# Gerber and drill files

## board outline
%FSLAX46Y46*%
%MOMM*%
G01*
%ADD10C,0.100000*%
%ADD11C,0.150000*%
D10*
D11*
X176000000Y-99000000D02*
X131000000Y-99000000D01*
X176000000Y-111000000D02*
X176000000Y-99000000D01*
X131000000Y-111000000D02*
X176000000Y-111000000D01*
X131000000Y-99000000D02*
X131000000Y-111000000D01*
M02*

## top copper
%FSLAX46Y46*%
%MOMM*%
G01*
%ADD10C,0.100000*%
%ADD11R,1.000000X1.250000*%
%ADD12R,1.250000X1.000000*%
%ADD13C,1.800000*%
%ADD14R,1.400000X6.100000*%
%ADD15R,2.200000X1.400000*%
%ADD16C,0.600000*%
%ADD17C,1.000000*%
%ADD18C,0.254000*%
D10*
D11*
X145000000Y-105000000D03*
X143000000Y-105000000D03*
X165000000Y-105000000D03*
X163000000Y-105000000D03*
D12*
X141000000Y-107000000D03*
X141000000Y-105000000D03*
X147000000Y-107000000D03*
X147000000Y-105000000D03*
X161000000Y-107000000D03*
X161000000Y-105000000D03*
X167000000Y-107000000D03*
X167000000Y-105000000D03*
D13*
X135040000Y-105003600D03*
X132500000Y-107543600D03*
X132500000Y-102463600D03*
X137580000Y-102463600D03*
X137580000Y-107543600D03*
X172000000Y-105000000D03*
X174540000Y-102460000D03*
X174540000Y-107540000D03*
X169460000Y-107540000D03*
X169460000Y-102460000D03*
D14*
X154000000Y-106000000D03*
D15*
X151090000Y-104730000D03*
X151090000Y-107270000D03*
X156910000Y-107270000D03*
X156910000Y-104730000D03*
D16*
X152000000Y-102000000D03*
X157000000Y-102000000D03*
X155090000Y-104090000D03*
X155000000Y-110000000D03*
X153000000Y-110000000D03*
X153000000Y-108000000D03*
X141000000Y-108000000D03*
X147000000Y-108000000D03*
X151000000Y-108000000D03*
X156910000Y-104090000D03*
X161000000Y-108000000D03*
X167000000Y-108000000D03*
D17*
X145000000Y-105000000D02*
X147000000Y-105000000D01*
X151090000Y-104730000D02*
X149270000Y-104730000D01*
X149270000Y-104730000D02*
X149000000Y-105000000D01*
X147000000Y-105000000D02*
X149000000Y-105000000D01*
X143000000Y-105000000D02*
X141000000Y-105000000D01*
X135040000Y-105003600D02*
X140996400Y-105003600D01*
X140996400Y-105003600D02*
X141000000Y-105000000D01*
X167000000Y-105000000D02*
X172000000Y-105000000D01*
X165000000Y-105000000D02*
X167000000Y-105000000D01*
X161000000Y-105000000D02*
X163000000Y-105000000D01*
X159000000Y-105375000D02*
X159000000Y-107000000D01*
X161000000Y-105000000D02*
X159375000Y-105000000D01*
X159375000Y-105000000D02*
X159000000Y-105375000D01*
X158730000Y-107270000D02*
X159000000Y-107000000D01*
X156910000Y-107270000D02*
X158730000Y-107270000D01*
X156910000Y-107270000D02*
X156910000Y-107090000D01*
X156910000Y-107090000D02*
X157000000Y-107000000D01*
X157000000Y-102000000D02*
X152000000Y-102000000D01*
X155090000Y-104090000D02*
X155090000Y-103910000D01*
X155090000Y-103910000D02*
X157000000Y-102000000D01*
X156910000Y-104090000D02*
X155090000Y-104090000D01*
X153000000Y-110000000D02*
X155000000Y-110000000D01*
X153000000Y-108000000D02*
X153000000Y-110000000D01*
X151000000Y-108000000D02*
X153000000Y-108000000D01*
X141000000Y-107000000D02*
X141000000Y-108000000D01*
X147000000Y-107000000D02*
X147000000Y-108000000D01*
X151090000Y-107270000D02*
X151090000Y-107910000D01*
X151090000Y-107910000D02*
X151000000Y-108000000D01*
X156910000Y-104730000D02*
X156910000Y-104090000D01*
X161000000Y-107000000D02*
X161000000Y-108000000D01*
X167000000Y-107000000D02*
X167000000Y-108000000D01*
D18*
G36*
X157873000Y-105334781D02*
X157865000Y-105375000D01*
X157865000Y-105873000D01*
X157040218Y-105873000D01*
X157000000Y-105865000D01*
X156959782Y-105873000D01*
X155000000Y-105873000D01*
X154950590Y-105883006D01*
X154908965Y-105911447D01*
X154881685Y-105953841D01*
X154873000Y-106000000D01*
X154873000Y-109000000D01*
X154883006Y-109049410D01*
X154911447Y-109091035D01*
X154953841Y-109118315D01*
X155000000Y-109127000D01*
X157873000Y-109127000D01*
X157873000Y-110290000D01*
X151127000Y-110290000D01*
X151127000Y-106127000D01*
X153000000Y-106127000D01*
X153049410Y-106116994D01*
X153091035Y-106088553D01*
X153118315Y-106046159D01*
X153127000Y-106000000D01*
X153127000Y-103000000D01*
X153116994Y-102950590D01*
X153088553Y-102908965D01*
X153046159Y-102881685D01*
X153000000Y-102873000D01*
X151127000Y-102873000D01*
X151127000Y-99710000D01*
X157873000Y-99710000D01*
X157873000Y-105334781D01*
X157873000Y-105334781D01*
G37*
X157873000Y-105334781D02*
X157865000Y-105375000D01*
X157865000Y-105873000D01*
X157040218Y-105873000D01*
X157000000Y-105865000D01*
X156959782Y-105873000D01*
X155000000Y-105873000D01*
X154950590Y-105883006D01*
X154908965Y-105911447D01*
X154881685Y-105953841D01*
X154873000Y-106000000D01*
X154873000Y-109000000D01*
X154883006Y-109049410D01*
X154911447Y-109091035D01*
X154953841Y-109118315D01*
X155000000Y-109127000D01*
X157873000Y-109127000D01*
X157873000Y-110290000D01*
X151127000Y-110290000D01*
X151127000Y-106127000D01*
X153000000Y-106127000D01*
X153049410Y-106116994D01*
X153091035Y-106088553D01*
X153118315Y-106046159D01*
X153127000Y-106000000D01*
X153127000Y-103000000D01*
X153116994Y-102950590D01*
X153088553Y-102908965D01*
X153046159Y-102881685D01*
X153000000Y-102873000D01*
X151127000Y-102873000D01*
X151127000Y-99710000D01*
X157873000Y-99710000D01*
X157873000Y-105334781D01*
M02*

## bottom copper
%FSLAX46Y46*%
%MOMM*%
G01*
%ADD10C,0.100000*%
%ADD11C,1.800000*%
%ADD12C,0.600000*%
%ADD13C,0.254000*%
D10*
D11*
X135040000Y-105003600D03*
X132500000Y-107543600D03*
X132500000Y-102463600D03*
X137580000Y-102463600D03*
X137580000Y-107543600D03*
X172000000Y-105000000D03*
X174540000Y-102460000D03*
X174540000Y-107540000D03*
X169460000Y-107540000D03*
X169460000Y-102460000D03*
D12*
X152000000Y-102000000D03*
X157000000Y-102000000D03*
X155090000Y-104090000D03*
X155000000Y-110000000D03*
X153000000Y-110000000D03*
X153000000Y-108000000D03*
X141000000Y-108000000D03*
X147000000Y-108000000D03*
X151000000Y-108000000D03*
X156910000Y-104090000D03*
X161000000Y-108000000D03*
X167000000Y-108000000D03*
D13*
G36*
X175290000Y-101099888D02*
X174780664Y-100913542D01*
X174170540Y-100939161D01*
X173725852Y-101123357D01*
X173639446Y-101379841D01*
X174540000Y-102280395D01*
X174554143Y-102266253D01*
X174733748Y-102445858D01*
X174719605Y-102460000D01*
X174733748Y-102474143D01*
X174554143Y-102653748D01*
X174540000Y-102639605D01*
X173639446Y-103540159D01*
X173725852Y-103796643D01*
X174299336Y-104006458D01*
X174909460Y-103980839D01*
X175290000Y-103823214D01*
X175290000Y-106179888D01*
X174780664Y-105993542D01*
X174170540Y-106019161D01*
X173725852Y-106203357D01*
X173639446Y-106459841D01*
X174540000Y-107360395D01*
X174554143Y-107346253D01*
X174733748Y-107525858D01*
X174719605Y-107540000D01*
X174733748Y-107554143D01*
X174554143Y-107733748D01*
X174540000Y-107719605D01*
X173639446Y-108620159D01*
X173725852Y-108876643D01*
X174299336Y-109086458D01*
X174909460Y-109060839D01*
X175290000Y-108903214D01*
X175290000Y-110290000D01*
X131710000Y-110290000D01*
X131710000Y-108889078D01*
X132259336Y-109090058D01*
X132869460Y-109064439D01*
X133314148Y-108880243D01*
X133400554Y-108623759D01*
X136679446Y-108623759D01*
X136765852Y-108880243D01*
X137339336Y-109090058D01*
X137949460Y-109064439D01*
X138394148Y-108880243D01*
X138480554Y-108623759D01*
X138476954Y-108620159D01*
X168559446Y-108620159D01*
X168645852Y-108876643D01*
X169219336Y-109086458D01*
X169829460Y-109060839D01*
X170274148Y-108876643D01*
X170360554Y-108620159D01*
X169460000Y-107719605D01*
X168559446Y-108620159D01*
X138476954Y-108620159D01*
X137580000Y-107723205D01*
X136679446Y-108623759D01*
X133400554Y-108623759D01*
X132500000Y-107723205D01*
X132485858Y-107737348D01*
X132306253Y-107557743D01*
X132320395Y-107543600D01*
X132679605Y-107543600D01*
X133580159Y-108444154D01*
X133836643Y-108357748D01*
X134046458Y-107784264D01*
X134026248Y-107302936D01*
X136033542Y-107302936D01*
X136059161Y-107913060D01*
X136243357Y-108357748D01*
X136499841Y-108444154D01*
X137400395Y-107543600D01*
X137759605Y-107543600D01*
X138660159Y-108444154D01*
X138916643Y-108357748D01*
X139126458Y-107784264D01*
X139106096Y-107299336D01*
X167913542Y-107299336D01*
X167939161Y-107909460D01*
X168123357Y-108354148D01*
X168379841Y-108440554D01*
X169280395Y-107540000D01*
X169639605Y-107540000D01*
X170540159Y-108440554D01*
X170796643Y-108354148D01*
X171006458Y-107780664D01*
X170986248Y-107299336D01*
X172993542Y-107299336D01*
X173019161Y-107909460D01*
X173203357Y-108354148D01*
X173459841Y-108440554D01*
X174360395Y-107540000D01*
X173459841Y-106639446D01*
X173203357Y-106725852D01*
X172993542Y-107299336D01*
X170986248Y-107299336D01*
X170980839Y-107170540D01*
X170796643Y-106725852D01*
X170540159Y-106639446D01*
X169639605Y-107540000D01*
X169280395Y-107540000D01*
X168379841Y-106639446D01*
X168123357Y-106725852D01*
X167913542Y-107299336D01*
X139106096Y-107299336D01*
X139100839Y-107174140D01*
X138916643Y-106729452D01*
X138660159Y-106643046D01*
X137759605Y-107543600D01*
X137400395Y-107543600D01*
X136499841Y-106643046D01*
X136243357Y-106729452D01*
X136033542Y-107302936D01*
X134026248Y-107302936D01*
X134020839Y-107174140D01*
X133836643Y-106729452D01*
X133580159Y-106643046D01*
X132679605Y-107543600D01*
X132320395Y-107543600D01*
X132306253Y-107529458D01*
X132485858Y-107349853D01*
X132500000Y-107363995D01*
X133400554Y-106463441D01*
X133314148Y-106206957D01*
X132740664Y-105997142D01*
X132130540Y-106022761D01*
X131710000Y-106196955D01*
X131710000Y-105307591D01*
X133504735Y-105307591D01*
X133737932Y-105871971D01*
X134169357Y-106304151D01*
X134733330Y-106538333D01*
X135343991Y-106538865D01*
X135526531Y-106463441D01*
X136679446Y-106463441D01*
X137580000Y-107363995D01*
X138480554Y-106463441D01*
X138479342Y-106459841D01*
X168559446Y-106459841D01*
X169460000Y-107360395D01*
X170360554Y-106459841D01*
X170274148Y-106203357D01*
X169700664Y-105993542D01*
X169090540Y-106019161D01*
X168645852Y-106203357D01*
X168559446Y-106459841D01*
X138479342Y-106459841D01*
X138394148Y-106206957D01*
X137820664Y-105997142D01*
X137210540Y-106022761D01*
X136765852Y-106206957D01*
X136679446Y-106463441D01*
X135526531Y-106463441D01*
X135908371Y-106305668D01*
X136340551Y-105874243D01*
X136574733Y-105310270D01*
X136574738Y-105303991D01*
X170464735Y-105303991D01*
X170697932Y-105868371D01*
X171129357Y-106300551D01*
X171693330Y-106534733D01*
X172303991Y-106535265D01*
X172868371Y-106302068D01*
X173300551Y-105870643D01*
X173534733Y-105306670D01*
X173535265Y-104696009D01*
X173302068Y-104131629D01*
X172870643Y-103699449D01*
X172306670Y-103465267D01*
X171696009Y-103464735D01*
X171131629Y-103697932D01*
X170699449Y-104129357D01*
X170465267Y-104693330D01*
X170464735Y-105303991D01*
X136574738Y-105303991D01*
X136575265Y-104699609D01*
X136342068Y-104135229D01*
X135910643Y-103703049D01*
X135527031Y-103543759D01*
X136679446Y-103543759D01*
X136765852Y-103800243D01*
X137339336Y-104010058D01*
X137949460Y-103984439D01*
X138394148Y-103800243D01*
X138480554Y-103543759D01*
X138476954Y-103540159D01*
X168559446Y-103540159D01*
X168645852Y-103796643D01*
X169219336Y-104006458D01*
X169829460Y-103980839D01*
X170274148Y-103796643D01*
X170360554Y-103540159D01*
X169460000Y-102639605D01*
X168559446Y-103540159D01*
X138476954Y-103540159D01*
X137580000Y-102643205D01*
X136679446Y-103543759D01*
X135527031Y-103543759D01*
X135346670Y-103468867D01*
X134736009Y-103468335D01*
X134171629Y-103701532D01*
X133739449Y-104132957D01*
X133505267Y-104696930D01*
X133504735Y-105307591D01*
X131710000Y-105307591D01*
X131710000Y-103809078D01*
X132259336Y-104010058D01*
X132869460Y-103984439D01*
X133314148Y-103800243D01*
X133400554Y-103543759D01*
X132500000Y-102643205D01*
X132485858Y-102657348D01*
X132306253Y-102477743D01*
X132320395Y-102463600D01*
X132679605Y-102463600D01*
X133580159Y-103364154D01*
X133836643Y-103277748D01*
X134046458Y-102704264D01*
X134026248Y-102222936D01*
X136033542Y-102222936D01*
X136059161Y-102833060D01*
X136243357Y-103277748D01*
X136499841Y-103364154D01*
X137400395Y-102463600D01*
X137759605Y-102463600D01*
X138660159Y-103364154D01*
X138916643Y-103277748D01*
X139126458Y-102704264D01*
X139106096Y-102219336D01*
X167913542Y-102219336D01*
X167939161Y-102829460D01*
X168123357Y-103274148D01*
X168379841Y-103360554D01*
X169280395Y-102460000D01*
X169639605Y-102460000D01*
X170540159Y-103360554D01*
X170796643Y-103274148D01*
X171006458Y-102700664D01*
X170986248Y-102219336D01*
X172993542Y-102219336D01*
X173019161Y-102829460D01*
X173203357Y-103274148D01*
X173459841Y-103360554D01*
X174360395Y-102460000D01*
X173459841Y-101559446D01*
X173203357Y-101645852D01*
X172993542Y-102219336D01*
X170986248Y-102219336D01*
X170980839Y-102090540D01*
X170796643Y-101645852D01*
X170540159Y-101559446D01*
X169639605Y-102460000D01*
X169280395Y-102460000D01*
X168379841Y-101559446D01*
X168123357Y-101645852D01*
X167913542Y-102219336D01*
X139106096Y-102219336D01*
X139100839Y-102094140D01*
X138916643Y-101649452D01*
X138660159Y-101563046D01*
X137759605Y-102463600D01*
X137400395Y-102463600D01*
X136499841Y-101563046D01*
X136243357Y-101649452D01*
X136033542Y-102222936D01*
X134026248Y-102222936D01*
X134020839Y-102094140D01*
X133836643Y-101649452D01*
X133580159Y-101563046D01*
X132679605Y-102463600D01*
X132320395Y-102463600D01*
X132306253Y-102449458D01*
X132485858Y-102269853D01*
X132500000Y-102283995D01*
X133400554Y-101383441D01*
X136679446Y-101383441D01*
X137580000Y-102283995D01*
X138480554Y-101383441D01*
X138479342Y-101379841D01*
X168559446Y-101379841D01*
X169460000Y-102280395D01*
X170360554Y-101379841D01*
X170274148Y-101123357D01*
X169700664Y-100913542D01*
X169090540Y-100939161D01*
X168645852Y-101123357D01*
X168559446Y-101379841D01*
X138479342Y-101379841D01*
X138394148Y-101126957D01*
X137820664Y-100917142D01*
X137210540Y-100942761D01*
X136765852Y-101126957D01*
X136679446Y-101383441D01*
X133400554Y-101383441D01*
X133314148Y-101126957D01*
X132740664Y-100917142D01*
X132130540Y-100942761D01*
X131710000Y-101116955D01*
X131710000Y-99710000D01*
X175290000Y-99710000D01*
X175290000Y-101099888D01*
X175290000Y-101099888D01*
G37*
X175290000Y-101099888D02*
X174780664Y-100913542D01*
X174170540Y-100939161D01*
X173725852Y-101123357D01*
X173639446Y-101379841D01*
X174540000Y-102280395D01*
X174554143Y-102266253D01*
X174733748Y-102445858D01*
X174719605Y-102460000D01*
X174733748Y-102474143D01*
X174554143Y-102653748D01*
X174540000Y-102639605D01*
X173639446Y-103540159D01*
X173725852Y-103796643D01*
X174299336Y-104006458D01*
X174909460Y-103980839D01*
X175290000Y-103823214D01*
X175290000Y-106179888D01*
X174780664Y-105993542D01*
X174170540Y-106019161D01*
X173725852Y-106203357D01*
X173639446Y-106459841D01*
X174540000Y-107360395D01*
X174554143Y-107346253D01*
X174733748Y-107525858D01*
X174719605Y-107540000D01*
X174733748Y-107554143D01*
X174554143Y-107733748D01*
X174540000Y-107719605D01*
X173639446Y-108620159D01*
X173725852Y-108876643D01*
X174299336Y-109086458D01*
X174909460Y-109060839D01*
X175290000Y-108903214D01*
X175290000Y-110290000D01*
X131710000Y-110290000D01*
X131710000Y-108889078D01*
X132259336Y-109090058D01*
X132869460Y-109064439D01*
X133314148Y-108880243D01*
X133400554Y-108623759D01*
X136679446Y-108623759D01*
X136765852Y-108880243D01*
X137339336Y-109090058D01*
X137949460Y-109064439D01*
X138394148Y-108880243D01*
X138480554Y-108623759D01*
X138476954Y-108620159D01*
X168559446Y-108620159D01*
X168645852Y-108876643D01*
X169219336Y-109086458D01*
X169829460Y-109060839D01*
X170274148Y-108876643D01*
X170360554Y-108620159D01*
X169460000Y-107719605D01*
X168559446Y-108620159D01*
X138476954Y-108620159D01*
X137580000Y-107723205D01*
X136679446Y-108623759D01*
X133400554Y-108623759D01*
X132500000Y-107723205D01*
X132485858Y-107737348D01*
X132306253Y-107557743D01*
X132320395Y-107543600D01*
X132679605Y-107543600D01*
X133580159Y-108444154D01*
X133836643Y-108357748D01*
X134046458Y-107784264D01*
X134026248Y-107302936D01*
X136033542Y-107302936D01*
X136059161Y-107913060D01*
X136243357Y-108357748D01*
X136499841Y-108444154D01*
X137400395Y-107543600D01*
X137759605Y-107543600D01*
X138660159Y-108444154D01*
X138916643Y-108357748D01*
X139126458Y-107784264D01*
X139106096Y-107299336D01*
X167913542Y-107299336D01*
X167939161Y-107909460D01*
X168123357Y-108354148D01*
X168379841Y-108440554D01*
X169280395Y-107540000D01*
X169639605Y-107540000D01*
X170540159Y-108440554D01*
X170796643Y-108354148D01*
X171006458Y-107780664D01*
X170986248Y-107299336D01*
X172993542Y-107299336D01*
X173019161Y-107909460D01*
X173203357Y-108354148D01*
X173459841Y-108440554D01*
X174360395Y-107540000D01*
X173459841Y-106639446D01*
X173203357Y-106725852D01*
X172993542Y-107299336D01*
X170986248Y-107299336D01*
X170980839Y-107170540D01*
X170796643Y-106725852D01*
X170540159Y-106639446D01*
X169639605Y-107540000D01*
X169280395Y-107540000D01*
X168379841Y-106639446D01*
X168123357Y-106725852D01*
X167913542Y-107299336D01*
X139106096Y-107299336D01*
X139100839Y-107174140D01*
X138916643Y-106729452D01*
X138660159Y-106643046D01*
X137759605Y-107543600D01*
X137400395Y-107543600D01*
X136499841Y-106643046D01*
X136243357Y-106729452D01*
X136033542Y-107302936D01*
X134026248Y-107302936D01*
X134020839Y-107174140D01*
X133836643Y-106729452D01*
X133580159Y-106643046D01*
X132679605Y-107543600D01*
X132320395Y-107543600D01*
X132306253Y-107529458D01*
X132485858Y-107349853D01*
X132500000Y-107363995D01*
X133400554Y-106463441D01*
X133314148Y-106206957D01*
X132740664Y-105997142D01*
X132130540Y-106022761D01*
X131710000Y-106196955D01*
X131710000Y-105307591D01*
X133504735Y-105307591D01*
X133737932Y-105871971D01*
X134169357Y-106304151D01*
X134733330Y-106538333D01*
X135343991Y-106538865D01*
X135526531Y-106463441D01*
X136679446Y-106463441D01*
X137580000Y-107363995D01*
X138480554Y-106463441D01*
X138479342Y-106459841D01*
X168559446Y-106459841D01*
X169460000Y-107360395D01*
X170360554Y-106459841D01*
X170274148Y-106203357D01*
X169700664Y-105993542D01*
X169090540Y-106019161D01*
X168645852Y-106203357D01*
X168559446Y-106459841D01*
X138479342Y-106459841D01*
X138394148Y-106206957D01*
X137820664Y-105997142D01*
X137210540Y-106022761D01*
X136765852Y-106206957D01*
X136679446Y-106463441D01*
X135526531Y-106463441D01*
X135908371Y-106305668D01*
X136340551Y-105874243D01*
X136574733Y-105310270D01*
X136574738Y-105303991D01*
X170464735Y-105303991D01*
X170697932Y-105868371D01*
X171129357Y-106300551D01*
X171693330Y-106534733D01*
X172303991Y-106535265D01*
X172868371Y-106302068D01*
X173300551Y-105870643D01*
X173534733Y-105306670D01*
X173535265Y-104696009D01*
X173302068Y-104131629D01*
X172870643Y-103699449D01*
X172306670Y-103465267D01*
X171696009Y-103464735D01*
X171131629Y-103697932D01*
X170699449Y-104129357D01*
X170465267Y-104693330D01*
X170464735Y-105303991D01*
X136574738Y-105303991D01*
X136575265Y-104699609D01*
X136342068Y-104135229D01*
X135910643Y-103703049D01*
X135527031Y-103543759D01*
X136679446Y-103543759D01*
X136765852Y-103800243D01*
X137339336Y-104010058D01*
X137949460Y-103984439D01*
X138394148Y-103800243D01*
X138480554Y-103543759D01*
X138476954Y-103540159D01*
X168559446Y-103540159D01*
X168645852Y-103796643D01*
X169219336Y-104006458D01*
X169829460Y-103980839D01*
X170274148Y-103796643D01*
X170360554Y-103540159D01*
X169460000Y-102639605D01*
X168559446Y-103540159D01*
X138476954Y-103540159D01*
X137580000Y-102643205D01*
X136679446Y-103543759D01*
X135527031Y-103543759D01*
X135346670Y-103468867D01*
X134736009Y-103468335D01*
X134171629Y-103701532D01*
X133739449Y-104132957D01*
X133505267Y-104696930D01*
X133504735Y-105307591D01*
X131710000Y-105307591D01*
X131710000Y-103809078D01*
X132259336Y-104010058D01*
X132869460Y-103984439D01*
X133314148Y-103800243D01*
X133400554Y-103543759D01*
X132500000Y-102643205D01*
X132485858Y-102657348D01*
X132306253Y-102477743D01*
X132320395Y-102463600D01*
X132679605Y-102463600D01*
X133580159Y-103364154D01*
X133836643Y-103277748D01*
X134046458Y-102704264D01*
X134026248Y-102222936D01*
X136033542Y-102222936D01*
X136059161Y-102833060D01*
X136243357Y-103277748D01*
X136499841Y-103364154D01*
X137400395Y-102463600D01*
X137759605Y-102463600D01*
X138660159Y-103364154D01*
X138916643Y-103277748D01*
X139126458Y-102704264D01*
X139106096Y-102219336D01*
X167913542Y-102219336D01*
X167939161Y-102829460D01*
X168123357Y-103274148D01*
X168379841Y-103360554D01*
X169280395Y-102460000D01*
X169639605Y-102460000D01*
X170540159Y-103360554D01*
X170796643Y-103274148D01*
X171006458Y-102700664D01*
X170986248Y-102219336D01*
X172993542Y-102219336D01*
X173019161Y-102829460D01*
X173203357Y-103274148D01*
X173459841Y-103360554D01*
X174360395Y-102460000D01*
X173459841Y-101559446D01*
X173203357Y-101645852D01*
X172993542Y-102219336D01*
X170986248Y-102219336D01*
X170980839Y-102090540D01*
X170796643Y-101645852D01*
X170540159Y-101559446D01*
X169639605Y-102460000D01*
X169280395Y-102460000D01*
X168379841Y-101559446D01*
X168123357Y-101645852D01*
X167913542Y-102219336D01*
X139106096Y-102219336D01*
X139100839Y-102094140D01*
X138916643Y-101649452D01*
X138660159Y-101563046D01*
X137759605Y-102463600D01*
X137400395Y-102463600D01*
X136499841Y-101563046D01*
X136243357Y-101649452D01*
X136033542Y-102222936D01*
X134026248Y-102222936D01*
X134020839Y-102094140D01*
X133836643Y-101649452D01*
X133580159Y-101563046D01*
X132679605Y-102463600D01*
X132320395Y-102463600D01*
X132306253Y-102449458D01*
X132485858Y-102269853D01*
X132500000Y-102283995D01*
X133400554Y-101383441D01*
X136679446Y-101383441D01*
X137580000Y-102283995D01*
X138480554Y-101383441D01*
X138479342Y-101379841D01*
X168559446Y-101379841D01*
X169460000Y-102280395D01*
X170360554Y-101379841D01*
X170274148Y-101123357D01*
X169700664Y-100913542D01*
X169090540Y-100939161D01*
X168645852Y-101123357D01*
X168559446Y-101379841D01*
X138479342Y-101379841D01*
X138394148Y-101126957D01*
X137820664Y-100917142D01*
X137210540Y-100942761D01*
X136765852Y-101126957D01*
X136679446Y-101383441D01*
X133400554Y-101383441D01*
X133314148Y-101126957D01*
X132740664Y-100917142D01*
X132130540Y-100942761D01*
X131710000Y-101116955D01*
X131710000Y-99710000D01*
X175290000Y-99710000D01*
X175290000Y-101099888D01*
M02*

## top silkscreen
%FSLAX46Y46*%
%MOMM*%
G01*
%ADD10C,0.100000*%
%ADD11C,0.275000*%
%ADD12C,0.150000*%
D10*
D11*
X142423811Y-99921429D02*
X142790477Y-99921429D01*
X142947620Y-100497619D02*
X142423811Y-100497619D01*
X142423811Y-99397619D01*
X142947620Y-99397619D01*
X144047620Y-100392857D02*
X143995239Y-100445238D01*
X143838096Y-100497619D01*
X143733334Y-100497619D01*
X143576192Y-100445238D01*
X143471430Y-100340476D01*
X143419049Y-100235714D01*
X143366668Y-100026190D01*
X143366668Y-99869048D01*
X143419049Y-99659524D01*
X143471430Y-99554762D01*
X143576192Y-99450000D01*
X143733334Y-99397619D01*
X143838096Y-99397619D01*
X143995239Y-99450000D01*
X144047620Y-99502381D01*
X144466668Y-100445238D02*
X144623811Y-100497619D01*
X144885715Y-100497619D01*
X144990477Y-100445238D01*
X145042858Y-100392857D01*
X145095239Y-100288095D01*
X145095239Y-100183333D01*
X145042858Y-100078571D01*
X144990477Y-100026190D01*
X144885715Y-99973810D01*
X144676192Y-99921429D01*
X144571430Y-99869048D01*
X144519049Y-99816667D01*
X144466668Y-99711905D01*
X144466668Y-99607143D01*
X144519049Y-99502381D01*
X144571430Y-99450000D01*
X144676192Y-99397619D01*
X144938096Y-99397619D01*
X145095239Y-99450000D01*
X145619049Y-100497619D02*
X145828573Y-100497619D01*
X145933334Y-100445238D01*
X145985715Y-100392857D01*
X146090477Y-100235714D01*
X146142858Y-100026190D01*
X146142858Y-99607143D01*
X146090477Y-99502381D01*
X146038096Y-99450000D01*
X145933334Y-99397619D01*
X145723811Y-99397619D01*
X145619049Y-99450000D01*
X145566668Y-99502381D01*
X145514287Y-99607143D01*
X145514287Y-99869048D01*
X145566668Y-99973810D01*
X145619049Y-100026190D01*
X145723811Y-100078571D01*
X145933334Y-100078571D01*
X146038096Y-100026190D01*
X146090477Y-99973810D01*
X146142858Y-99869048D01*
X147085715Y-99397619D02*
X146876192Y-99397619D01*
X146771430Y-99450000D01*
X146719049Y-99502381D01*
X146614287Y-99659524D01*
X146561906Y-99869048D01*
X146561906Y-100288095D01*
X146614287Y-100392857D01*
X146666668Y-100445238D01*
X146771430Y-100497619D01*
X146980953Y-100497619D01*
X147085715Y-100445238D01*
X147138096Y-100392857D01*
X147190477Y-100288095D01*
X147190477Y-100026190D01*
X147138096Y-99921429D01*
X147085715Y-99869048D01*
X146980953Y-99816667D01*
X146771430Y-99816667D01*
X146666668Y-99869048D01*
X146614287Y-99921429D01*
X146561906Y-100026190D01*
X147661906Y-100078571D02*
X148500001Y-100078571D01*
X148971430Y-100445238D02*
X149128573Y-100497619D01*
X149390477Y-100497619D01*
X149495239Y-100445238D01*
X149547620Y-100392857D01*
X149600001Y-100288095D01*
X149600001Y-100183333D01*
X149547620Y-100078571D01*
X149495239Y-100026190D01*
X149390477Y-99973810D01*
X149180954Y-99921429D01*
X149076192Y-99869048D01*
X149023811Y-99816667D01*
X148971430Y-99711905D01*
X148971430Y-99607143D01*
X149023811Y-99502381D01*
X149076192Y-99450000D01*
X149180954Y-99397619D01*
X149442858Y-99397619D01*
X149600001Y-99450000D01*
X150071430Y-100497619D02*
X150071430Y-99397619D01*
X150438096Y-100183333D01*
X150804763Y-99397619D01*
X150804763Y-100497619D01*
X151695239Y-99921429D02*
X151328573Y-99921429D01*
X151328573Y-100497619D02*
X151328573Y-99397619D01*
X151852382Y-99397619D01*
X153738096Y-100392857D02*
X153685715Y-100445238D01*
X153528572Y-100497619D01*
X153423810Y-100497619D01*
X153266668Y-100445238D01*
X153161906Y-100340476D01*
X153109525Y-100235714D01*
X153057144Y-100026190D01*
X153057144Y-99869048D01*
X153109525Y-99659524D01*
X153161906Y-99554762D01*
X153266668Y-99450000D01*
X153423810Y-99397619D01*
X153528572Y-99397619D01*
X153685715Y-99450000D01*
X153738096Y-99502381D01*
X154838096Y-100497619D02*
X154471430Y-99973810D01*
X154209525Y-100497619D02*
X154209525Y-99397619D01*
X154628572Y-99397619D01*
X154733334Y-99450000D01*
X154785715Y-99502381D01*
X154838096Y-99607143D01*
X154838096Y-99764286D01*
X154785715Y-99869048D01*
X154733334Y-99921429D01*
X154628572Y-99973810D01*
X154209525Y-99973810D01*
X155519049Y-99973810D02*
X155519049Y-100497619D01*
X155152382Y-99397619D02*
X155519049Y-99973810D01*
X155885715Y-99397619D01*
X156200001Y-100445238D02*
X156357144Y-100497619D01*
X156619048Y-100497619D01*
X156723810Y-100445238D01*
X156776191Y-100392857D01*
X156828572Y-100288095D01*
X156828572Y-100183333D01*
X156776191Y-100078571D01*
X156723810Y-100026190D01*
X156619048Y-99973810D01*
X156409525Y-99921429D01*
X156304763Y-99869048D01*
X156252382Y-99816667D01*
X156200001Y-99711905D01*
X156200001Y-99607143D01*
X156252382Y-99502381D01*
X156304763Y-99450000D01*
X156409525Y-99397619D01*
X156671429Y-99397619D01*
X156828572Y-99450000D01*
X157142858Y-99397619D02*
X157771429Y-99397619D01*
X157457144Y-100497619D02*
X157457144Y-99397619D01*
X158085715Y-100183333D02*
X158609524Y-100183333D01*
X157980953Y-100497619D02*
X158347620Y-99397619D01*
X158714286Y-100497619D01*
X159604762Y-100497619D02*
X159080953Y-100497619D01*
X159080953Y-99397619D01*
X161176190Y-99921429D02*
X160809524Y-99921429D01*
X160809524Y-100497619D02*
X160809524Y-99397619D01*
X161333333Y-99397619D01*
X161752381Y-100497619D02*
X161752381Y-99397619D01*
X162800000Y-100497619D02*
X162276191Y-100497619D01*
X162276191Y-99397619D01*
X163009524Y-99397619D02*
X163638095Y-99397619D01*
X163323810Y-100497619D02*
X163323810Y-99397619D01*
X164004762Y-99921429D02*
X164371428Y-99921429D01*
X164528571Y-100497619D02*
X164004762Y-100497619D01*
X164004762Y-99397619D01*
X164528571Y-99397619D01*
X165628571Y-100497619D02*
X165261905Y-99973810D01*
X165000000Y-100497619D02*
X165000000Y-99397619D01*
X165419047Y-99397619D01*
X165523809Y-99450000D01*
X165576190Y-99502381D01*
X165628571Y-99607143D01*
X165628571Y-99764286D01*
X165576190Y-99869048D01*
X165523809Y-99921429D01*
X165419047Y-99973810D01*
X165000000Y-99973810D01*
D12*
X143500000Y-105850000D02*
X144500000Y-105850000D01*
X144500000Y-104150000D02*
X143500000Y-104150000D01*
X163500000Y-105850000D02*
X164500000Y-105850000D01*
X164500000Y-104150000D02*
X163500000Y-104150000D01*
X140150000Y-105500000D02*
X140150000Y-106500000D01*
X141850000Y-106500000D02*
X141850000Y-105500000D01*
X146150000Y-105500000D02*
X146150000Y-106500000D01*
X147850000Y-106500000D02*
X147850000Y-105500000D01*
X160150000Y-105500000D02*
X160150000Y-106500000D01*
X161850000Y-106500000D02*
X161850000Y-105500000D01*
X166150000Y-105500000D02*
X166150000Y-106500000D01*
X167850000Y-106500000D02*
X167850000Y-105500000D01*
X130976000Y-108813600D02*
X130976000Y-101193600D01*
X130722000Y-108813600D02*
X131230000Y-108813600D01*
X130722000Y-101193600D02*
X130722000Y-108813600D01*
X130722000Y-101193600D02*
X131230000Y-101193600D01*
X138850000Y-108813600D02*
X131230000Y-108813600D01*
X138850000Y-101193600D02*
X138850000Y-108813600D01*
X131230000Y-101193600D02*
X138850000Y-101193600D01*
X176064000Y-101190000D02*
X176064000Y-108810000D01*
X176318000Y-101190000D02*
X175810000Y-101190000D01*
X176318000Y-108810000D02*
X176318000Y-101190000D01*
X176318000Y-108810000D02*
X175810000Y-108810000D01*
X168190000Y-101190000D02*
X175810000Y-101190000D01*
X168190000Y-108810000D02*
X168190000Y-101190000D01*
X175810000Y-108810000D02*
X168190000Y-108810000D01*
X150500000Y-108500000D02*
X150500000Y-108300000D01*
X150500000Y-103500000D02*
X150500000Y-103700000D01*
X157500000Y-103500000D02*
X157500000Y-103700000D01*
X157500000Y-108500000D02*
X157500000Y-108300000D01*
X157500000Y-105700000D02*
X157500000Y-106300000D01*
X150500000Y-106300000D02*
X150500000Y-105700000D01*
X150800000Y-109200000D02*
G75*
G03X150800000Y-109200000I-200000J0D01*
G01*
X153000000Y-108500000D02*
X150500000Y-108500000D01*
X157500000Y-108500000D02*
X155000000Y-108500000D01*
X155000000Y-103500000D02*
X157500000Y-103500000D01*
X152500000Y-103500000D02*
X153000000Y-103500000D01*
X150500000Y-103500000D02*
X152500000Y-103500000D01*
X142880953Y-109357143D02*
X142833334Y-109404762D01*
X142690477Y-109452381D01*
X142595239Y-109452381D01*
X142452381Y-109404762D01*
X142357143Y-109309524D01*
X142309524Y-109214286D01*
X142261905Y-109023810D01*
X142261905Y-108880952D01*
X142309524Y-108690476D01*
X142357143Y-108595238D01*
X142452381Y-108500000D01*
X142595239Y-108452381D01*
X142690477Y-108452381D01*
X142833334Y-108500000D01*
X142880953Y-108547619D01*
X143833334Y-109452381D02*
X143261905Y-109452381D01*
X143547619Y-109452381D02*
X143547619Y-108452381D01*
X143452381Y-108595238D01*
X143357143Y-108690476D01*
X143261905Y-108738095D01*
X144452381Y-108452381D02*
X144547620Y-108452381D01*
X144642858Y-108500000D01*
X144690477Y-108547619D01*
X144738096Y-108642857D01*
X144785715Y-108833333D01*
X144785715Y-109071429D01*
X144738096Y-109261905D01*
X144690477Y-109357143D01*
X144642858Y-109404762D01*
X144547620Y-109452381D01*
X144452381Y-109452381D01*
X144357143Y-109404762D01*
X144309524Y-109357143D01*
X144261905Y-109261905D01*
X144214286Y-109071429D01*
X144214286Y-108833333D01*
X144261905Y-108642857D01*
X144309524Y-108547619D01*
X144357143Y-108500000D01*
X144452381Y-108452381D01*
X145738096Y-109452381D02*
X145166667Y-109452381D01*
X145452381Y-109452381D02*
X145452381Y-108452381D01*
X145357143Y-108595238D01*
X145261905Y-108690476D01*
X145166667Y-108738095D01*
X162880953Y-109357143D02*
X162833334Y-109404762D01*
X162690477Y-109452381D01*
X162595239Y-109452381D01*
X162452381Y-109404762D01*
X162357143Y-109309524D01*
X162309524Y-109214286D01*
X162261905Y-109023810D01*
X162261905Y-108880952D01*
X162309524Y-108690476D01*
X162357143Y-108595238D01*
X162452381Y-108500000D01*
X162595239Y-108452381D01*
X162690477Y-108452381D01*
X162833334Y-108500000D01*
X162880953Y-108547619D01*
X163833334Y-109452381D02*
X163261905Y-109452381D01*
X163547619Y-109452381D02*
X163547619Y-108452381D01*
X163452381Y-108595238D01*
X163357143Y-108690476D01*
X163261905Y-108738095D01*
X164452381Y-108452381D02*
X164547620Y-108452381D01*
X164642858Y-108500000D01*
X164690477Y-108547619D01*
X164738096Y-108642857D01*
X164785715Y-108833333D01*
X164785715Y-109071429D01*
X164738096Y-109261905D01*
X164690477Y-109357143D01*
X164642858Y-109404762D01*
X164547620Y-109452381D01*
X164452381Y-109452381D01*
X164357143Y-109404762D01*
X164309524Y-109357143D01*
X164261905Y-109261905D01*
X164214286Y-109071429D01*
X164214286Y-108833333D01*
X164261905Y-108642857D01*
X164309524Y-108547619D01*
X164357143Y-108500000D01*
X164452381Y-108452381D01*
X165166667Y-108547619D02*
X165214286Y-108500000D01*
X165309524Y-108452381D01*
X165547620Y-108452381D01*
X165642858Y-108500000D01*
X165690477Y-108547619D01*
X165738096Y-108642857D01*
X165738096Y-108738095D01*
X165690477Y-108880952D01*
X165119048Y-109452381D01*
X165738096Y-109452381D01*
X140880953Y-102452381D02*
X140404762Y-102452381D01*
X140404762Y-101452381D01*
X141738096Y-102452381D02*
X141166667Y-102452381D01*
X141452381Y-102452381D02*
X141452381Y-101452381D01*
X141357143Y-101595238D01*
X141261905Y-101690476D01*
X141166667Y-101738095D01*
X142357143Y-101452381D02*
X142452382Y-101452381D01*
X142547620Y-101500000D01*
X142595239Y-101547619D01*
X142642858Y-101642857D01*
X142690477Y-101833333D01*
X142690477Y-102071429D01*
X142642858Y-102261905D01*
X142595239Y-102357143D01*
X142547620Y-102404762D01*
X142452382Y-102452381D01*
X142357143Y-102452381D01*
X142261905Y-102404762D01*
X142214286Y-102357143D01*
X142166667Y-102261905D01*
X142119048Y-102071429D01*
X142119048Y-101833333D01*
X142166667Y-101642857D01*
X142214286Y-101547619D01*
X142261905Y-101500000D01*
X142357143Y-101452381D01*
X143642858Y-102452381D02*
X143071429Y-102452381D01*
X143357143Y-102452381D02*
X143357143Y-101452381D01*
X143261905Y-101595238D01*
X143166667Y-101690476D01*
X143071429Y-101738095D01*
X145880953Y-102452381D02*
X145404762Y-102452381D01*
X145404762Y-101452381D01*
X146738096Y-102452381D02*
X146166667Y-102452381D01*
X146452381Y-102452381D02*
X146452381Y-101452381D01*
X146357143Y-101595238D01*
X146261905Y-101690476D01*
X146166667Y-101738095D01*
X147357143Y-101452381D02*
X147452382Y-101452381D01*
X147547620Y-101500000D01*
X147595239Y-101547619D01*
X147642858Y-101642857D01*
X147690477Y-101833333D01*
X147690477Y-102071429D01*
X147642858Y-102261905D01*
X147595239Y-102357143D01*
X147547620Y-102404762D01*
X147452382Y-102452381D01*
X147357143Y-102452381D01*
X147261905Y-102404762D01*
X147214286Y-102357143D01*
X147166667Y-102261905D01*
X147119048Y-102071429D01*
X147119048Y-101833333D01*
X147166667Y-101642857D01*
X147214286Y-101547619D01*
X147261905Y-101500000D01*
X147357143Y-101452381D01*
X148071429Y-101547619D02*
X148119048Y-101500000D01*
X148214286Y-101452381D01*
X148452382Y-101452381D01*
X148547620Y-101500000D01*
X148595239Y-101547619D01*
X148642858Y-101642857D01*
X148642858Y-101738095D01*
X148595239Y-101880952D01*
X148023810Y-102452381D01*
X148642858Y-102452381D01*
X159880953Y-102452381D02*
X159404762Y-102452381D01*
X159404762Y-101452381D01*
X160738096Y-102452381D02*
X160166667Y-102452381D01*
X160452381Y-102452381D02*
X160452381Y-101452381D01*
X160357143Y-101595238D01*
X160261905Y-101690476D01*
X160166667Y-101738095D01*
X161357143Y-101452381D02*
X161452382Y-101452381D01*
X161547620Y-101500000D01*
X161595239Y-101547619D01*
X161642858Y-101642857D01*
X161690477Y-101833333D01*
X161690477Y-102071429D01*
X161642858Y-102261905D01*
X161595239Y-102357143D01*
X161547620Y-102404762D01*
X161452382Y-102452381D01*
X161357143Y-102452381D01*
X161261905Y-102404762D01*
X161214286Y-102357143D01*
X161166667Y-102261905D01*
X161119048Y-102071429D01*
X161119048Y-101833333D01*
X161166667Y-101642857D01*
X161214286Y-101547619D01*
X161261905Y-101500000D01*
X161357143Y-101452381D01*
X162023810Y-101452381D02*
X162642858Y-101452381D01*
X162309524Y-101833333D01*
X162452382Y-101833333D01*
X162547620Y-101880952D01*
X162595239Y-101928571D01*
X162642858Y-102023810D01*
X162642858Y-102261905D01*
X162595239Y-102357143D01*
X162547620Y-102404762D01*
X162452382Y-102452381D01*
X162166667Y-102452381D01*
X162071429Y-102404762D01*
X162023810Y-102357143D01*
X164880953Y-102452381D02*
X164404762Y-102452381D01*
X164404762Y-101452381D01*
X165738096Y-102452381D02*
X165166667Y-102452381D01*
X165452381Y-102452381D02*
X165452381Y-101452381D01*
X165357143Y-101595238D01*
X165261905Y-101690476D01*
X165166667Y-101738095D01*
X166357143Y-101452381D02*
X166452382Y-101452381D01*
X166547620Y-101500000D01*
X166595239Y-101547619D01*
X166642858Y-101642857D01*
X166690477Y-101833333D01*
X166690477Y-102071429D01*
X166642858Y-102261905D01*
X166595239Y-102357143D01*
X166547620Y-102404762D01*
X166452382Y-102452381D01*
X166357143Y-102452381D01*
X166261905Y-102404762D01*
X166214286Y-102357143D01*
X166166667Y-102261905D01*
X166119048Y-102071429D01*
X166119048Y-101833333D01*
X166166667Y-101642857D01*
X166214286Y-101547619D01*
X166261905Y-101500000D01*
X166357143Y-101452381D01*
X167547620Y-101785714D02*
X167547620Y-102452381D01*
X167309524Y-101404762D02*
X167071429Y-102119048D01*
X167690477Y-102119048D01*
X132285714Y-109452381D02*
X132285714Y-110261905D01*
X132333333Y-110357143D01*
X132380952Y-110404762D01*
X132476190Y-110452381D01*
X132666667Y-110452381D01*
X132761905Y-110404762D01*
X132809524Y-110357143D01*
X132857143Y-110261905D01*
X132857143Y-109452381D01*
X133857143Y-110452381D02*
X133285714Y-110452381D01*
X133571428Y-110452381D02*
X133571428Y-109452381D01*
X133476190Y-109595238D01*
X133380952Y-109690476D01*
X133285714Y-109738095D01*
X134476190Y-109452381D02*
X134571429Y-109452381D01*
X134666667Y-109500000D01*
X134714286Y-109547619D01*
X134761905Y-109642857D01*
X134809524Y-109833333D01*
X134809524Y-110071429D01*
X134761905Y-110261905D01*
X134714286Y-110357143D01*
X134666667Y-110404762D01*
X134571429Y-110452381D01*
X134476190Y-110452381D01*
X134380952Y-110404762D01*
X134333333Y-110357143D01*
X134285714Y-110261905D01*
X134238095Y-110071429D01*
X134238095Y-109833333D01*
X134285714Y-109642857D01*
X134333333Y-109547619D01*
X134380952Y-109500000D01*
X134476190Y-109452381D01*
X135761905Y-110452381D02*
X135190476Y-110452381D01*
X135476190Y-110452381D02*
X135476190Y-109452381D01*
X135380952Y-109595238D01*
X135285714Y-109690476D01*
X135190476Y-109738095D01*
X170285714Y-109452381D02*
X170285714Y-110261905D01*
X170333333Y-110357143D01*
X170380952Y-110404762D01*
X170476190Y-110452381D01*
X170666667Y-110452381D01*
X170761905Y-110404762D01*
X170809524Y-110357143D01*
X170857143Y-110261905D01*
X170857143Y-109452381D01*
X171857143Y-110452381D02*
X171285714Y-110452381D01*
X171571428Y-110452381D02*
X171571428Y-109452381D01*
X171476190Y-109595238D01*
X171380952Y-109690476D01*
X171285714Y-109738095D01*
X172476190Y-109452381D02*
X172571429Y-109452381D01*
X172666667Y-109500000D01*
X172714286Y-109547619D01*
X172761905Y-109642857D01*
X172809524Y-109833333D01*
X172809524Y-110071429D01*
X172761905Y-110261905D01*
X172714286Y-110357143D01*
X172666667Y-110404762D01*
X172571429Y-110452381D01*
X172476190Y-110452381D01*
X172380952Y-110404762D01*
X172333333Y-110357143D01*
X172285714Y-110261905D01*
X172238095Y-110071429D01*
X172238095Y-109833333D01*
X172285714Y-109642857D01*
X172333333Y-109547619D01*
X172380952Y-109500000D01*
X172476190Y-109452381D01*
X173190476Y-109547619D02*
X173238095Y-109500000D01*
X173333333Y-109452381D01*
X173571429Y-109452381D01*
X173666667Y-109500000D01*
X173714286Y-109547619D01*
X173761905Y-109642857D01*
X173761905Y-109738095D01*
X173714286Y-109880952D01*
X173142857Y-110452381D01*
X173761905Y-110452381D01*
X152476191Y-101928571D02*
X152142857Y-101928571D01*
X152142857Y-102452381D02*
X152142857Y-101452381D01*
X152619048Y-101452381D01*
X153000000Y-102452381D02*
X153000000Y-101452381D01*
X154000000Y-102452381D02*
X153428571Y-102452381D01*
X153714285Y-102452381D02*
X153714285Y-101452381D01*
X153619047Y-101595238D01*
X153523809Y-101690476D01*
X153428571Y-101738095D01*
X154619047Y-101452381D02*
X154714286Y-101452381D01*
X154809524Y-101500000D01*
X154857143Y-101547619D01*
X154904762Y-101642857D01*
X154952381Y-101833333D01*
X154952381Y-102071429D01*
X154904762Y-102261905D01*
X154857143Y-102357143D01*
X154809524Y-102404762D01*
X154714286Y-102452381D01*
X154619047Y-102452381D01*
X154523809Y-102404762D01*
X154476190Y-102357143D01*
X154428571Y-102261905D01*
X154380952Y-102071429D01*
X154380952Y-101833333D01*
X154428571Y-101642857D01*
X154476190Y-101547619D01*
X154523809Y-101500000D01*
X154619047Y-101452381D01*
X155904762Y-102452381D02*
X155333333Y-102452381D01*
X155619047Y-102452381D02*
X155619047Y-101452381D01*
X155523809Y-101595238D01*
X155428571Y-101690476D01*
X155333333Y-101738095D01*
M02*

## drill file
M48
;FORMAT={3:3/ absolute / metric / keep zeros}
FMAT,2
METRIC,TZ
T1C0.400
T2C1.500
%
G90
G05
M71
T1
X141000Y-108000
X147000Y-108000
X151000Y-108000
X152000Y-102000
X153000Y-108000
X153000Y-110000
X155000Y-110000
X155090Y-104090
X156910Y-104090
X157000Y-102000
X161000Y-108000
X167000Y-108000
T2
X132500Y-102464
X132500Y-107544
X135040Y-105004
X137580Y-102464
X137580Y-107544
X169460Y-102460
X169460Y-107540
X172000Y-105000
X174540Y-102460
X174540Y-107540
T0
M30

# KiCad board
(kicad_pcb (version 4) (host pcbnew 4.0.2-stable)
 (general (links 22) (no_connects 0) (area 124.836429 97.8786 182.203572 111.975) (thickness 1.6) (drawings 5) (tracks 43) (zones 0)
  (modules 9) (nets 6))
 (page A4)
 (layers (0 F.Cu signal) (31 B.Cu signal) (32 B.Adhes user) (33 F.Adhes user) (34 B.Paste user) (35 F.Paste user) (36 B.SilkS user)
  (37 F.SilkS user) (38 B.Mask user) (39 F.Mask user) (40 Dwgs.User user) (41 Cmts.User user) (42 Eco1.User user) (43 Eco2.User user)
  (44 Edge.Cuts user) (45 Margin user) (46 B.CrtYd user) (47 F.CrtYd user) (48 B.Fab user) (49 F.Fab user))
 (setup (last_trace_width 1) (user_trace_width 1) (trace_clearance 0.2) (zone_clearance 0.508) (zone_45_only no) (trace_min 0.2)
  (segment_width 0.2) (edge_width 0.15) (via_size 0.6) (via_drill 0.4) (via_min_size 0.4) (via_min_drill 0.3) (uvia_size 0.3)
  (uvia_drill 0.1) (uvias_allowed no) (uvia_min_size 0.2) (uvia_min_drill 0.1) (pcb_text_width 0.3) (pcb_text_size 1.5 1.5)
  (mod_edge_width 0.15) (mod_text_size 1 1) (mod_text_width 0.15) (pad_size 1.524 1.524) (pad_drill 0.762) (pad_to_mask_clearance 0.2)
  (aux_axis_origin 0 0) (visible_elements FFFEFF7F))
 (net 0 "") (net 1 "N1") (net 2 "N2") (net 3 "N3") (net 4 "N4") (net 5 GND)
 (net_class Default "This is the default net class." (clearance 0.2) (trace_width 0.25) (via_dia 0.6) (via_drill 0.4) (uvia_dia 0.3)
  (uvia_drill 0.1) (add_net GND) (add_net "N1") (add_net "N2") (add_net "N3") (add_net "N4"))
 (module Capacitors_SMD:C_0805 (layer F.Cu) (at 144 105 180)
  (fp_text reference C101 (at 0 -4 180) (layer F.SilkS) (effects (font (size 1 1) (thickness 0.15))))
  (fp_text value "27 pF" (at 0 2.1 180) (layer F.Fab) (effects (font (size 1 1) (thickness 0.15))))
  (fp_line (start 0.5 -0.85) (end -0.5 -0.85) (layer F.SilkS) (width 0.15))
  (fp_line (start -0.5 0.85) (end 0.5 0.85) (layer F.SilkS) (width 0.15))
  (pad 1 smd rect (at -1 0 180) (size 1 1.25) (layers F.Cu F.Paste F.Mask) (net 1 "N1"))
  (pad 2 smd rect (at 1 0 180) (size 1 1.25) (layers F.Cu F.Paste F.Mask) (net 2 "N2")))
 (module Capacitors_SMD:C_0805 (layer F.Cu) (at 164 105 180)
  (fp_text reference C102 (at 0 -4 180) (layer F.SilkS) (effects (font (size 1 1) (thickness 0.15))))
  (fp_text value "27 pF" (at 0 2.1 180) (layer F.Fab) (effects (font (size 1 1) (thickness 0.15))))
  (fp_line (start 0.5 -0.85) (end -0.5 -0.85) (layer F.SilkS) (width 0.15))
  (fp_line (start -0.5 0.85) (end 0.5 0.85) (layer F.SilkS) (width 0.15))
  (pad 1 smd rect (at -1 0 180) (size 1 1.25) (layers F.Cu F.Paste F.Mask) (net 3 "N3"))
  (pad 2 smd rect (at 1 0 180) (size 1 1.25) (layers F.Cu F.Paste F.Mask) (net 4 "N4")))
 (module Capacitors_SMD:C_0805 (layer F.Cu) (at 141 106 90)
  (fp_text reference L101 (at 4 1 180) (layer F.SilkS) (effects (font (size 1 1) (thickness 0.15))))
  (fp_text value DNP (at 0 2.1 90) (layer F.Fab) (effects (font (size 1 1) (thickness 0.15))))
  (fp_line (start 0.5 -0.85) (end -0.5 -0.85) (layer F.SilkS) (width 0.15))
  (fp_line (start -0.5 0.85) (end 0.5 0.85) (layer F.SilkS) (width 0.15))
  (pad 1 smd rect (at -1 0 90) (size 1 1.25) (layers F.Cu F.Paste F.Mask) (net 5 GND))
  (pad 2 smd rect (at 1 0 90) (size 1 1.25) (layers F.Cu F.Paste F.Mask) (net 2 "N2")))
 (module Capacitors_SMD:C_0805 (layer F.Cu) (at 147 106 90)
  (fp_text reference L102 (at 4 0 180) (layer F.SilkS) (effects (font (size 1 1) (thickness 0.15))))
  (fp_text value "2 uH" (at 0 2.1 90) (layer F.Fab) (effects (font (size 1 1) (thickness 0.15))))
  (fp_line (start 0.5 -0.85) (end -0.5 -0.85) (layer F.SilkS) (width 0.15))
  (fp_line (start -0.5 0.85) (end 0.5 0.85) (layer F.SilkS) (width 0.15))
  (pad 1 smd rect (at -1 0 90) (size 1 1.25) (layers F.Cu F.Paste F.Mask) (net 5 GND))
  (pad 2 smd rect (at 1 0 90) (size 1 1.25) (layers F.Cu F.Paste F.Mask) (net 1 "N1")))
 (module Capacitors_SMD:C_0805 (layer F.Cu) (at 161 106 90)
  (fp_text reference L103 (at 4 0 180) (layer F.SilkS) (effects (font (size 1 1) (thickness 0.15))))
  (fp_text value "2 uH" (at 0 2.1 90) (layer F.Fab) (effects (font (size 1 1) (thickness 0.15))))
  (fp_line (start 0.5 -0.85) (end -0.5 -0.85) (layer F.SilkS) (width 0.15))
  (fp_line (start -0.5 0.85) (end 0.5 0.85) (layer F.SilkS) (width 0.15))
  (pad 1 smd rect (at -1 0 90) (size 1 1.25) (layers F.Cu F.Paste F.Mask) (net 5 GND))
  (pad 2 smd rect (at 1 0 90) (size 1 1.25) (layers F.Cu F.Paste F.Mask) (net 4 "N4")))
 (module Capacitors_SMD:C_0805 (layer F.Cu) (at 167 106 90)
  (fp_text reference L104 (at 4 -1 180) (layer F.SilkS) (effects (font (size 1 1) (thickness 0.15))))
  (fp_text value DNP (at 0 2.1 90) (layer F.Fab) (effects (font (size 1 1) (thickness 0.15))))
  (fp_line (start 0.5 -0.85) (end -0.5 -0.85) (layer F.SilkS) (width 0.15))
  (fp_line (start -0.5 0.85) (end 0.5 0.85) (layer F.SilkS) (width 0.15))
  (pad 1 smd rect (at -1 0 90) (size 1 1.25) (layers F.Cu F.Paste F.Mask) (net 5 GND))
  (pad 2 smd rect (at 1 0 90) (size 1 1.25) (layers F.Cu F.Paste F.Mask) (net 3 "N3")))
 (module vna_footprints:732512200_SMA (layer F.Cu) (at 135.04 105.0036)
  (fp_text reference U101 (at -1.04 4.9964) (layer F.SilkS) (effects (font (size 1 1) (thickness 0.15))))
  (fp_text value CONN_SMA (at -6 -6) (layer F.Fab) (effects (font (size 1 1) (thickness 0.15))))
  (fp_line (start -4.064 3.81) (end -4.064 -3.81) (layer F.SilkS) (width 0.15))
  (fp_line (start -4.318 3.81) (end -3.81 3.81) (layer F.SilkS) (width 0.15))
  (fp_line (start -4.318 -3.81) (end -4.318 3.81) (layer F.SilkS) (width 0.15))
  (fp_line (start -4.318 -3.81) (end -3.81 -3.81) (layer F.SilkS) (width 0.15))
  (fp_line (start 3.81 3.81) (end -3.81 3.81) (layer F.SilkS) (width 0.15))
  (fp_line (start 3.81 -3.81) (end 3.81 3.81) (layer F.SilkS) (width 0.15))
  (fp_line (start -3.81 -3.81) (end 3.81 -3.81) (layer F.SilkS) (width 0.15))
  (pad 1 thru_hole circle (at 0 0) (size 1.8 1.8) (drill 1.5) (layers *.Cu *.Mask F.SilkS) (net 2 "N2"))
  (pad 2 thru_hole circle (at -2.54 2.54) (size 1.8 1.8) (drill 1.5) (layers *.Cu *.Mask F.SilkS) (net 5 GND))
  (pad 3 thru_hole circle (at -2.54 -2.54) (size 1.8 1.8) (drill 1.5) (layers *.Cu *.Mask F.SilkS) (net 5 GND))
  (pad 4 thru_hole circle (at 2.54 -2.54) (size 1.8 1.8) (drill 1.5) (layers *.Cu *.Mask F.SilkS) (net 5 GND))
  (pad 5 thru_hole circle (at 2.54 2.54) (size 1.8 1.8) (drill 1.5) (layers *.Cu *.Mask F.SilkS) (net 5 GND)))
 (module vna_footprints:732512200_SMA (layer F.Cu) (at 172 105 180)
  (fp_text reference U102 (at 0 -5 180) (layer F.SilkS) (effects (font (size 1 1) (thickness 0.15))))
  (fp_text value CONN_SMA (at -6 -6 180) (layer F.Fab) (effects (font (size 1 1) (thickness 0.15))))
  (fp_line (start -4.064 3.81) (end -4.064 -3.81) (layer F.SilkS) (width 0.15))
  (fp_line (start -4.318 3.81) (end -3.81 3.81) (layer F.SilkS) (width 0.15))
  (fp_line (start -4.318 -3.81) (end -4.318 3.81) (layer F.SilkS) (width 0.15))
  (fp_line (start -4.318 -3.81) (end -3.81 -3.81) (layer F.SilkS) (width 0.15))
  (fp_line (start 3.81 3.81) (end -3.81 3.81) (layer F.SilkS) (width 0.15))
  (fp_line (start 3.81 -3.81) (end 3.81 3.81) (layer F.SilkS) (width 0.15))
  (fp_line (start -3.81 -3.81) (end 3.81 -3.81) (layer F.SilkS) (width 0.15))
  (pad 1 thru_hole circle (at 0 0 180) (size 1.8 1.8) (drill 1.5) (layers *.Cu *.Mask F.SilkS) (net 3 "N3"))
  (pad 2 thru_hole circle (at -2.54 2.54 180) (size 1.8 1.8) (drill 1.5) (layers *.Cu *.Mask F.SilkS) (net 5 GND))
  (pad 3 thru_hole circle (at -2.54 -2.54 180) (size 1.8 1.8) (drill 1.5) (layers *.Cu *.Mask F.SilkS) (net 5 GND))
  (pad 4 thru_hole circle (at 2.54 -2.54 180) (size 1.8 1.8) (drill 1.5) (layers *.Cu *.Mask F.SilkS) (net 5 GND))
  (pad 5 thru_hole circle (at 2.54 2.54 180) (size 1.8 1.8) (drill 1.5) (layers *.Cu *.Mask F.SilkS) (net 5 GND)))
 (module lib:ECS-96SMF (layer F.Cu) (at 154 106)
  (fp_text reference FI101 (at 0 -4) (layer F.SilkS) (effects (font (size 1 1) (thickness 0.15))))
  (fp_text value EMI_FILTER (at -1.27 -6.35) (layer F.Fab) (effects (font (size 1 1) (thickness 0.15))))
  (fp_line (start -3.5 2.5) (end -3.5 2.3) (layer F.SilkS) (width 0.15))
  (fp_line (start -3.5 -2.5) (end -3.5 -2.3) (layer F.SilkS) (width 0.15))
  (fp_line (start 3.5 -2.5) (end 3.5 -2.3) (layer F.SilkS) (width 0.15))
  (fp_line (start 3.5 2.5) (end 3.5 2.3) (layer F.SilkS) (width 0.15))
  (fp_line (start 3.5 -0.3) (end 3.5 0.3) (layer F.SilkS) (width 0.15))
  (fp_line (start -3.5 0.3) (end -3.5 -0.3) (layer F.SilkS) (width 0.15))
  (fp_circle (center -3.4 3.2) (end -3.6 3.2) (layer F.SilkS) (width 0.15))
  (fp_line (start -1 2.5) (end -3.5 2.5) (layer F.SilkS) (width 0.15))
  (fp_line (start 3.5 2.5) (end 1 2.5) (layer F.SilkS) (width 0.15))
  (fp_line (start 1 -2.5) (end 3.5 -2.5) (layer F.SilkS) (width 0.15))
  (fp_line (start -1.5 -2.5) (end -1 -2.5) (layer F.SilkS) (width 0.15))
  (fp_line (start -3.5 -2.5) (end -1.5 -2.5) (layer F.SilkS) (width 0.15))
  (pad 2 smd rect (at 0 0) (size 1.4 6.1) (layers F.Cu F.Paste F.Mask) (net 5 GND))
  (pad 1 smd rect (at -2.91 -1.27) (size 2.2 1.4) (layers F.Cu F.Paste F.Mask) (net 1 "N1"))
  (pad 2 smd rect (at -2.91 1.27) (size 2.2 1.4) (layers F.Cu F.Paste F.Mask) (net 5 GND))
  (pad 3 smd rect (at 2.91 1.27) (size 2.2 1.4) (layers F.Cu F.Paste F.Mask) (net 4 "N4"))
  (pad 2 smd rect (at 2.91 -1.27) (size 2.2 1.4) (layers F.Cu F.Paste F.Mask) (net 5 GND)))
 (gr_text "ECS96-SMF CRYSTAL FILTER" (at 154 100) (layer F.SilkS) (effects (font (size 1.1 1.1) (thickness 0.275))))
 (gr_line (start 176 99) (end 131 99) (layer Edge.Cuts) (width 0.15))
 (gr_line (start 176 111) (end 176 99) (layer Edge.Cuts) (width 0.15))
 (gr_line (start 131 111) (end 176 111) (layer Edge.Cuts) (width 0.15))
 (gr_line (start 131 99) (end 131 111) (layer Edge.Cuts) (width 0.15))
 (segment (start 145 105) (end 147 105) (width 1) (layer F.Cu) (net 1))
 (segment (start 151.09 104.73) (end 149.27 104.73) (width 1) (layer F.Cu) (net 1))
 (segment (start 149.27 104.73) (end 149 105) (width 1) (layer F.Cu) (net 1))
 (segment (start 147 105) (end 149 105) (width 1) (layer F.Cu) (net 1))
 (segment (start 143 105) (end 141 105) (width 1) (layer F.Cu) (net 2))
 (segment (start 135.04 105.0036) (end 140.9964 105.0036) (width 1) (layer F.Cu) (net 2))
 (segment (start 140.9964 105.0036) (end 141 105) (width 1) (layer F.Cu) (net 2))
 (segment (start 167 105) (end 172 105) (width 1) (layer F.Cu) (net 3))
 (segment (start 165 105) (end 167 105) (width 1) (layer F.Cu) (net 3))
 (segment (start 161 105) (end 163 105) (width 1) (layer F.Cu) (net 4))
 (segment (start 159 105.375) (end 159 107) (width 1) (layer F.Cu) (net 4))
 (segment (start 161 105) (end 159.375 105) (width 1) (layer F.Cu) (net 4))
 (segment (start 159.375 105) (end 159 105.375) (width 1) (layer F.Cu) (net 4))
 (segment (start 158.73 107.27) (end 159 107) (width 1) (layer F.Cu) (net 4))
 (segment (start 156.91 107.27) (end 158.73 107.27) (width 1) (layer F.Cu) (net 4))
 (segment (start 156.91 107.27) (end 156.91 107.09) (width 1) (layer F.Cu) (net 4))
 (segment (start 156.91 107.09) (end 157 107) (width 1) (layer F.Cu) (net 4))
 (segment (start 157 102) (end 152 102) (width 1) (layer F.Cu) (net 5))
 (via (at 152 102) (size 0.6) (drill 0.4) (layers F.Cu B.Cu) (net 5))
 (segment (start 155.09 104.09) (end 155.09 103.91) (width 1) (layer F.Cu) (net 5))
 (segment (start 155.09 103.91) (end 157 102) (width 1) (layer F.Cu) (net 5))
 (via (at 157 102) (size 0.6) (drill 0.4) (layers F.Cu B.Cu) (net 5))
 (via (at 155.09 104.09) (size 0.6) (drill 0.4) (layers F.Cu B.Cu) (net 5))
 (segment (start 156.91 104.09) (end 155.09 104.09) (width 1) (layer F.Cu) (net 5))
 (segment (start 153 110) (end 155 110) (width 1) (layer F.Cu) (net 5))
 (via (at 155 110) (size 0.6) (drill 0.4) (layers F.Cu B.Cu) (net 5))
 (via (at 153 110) (size 0.6) (drill 0.4) (layers F.Cu B.Cu) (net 5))
 (segment (start 153 108) (end 153 110) (width 1) (layer F.Cu) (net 5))
 (via (at 153 108) (size 0.6) (drill 0.4) (layers F.Cu B.Cu) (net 5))
 (segment (start 151 108) (end 153 108) (width 1) (layer F.Cu) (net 5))
 (via (at 141 108) (size 0.6) (drill 0.4) (layers F.Cu B.Cu) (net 5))
 (segment (start 141 107) (end 141 108) (width 1) (layer F.Cu) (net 5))
 (via (at 147 108) (size 0.6) (drill 0.4) (layers F.Cu B.Cu) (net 5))
 (segment (start 147 107) (end 147 108) (width 1) (layer F.Cu) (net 5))
 (segment (start 151.09 107.27) (end 151.09 107.91) (width 1) (layer F.Cu) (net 5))
 (segment (start 151.09 107.91) (end 151 108) (width 1) (layer F.Cu) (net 5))
 (via (at 151 108) (size 0.6) (drill 0.4) (layers F.Cu B.Cu) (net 5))
 (via (at 156.91 104.09) (size 0.6) (drill 0.4) (layers F.Cu B.Cu) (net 5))
 (segment (start 156.91 104.73) (end 156.91 104.09) (width 1) (layer F.Cu) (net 5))
 (via (at 161 108) (size 0.6) (drill 0.4) (layers F.Cu B.Cu) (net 5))
 (segment (start 161 107) (end 161 108) (width 1) (layer F.Cu) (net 5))
 (via (at 167 108) (size 0.6) (drill 0.4) (layers F.Cu B.Cu) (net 5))
 (segment (start 167 107) (end 167 108) (width 1) (layer F.Cu) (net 5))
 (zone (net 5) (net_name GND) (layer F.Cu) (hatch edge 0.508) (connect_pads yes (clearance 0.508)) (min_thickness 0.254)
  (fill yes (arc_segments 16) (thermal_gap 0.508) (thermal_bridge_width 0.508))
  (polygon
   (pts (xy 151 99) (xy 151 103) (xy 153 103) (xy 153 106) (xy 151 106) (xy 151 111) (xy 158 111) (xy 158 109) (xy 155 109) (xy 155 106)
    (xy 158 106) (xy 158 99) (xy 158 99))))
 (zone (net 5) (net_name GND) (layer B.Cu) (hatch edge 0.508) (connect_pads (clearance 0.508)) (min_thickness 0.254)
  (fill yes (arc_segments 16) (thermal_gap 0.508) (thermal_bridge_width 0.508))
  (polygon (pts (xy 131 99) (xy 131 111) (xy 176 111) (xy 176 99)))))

